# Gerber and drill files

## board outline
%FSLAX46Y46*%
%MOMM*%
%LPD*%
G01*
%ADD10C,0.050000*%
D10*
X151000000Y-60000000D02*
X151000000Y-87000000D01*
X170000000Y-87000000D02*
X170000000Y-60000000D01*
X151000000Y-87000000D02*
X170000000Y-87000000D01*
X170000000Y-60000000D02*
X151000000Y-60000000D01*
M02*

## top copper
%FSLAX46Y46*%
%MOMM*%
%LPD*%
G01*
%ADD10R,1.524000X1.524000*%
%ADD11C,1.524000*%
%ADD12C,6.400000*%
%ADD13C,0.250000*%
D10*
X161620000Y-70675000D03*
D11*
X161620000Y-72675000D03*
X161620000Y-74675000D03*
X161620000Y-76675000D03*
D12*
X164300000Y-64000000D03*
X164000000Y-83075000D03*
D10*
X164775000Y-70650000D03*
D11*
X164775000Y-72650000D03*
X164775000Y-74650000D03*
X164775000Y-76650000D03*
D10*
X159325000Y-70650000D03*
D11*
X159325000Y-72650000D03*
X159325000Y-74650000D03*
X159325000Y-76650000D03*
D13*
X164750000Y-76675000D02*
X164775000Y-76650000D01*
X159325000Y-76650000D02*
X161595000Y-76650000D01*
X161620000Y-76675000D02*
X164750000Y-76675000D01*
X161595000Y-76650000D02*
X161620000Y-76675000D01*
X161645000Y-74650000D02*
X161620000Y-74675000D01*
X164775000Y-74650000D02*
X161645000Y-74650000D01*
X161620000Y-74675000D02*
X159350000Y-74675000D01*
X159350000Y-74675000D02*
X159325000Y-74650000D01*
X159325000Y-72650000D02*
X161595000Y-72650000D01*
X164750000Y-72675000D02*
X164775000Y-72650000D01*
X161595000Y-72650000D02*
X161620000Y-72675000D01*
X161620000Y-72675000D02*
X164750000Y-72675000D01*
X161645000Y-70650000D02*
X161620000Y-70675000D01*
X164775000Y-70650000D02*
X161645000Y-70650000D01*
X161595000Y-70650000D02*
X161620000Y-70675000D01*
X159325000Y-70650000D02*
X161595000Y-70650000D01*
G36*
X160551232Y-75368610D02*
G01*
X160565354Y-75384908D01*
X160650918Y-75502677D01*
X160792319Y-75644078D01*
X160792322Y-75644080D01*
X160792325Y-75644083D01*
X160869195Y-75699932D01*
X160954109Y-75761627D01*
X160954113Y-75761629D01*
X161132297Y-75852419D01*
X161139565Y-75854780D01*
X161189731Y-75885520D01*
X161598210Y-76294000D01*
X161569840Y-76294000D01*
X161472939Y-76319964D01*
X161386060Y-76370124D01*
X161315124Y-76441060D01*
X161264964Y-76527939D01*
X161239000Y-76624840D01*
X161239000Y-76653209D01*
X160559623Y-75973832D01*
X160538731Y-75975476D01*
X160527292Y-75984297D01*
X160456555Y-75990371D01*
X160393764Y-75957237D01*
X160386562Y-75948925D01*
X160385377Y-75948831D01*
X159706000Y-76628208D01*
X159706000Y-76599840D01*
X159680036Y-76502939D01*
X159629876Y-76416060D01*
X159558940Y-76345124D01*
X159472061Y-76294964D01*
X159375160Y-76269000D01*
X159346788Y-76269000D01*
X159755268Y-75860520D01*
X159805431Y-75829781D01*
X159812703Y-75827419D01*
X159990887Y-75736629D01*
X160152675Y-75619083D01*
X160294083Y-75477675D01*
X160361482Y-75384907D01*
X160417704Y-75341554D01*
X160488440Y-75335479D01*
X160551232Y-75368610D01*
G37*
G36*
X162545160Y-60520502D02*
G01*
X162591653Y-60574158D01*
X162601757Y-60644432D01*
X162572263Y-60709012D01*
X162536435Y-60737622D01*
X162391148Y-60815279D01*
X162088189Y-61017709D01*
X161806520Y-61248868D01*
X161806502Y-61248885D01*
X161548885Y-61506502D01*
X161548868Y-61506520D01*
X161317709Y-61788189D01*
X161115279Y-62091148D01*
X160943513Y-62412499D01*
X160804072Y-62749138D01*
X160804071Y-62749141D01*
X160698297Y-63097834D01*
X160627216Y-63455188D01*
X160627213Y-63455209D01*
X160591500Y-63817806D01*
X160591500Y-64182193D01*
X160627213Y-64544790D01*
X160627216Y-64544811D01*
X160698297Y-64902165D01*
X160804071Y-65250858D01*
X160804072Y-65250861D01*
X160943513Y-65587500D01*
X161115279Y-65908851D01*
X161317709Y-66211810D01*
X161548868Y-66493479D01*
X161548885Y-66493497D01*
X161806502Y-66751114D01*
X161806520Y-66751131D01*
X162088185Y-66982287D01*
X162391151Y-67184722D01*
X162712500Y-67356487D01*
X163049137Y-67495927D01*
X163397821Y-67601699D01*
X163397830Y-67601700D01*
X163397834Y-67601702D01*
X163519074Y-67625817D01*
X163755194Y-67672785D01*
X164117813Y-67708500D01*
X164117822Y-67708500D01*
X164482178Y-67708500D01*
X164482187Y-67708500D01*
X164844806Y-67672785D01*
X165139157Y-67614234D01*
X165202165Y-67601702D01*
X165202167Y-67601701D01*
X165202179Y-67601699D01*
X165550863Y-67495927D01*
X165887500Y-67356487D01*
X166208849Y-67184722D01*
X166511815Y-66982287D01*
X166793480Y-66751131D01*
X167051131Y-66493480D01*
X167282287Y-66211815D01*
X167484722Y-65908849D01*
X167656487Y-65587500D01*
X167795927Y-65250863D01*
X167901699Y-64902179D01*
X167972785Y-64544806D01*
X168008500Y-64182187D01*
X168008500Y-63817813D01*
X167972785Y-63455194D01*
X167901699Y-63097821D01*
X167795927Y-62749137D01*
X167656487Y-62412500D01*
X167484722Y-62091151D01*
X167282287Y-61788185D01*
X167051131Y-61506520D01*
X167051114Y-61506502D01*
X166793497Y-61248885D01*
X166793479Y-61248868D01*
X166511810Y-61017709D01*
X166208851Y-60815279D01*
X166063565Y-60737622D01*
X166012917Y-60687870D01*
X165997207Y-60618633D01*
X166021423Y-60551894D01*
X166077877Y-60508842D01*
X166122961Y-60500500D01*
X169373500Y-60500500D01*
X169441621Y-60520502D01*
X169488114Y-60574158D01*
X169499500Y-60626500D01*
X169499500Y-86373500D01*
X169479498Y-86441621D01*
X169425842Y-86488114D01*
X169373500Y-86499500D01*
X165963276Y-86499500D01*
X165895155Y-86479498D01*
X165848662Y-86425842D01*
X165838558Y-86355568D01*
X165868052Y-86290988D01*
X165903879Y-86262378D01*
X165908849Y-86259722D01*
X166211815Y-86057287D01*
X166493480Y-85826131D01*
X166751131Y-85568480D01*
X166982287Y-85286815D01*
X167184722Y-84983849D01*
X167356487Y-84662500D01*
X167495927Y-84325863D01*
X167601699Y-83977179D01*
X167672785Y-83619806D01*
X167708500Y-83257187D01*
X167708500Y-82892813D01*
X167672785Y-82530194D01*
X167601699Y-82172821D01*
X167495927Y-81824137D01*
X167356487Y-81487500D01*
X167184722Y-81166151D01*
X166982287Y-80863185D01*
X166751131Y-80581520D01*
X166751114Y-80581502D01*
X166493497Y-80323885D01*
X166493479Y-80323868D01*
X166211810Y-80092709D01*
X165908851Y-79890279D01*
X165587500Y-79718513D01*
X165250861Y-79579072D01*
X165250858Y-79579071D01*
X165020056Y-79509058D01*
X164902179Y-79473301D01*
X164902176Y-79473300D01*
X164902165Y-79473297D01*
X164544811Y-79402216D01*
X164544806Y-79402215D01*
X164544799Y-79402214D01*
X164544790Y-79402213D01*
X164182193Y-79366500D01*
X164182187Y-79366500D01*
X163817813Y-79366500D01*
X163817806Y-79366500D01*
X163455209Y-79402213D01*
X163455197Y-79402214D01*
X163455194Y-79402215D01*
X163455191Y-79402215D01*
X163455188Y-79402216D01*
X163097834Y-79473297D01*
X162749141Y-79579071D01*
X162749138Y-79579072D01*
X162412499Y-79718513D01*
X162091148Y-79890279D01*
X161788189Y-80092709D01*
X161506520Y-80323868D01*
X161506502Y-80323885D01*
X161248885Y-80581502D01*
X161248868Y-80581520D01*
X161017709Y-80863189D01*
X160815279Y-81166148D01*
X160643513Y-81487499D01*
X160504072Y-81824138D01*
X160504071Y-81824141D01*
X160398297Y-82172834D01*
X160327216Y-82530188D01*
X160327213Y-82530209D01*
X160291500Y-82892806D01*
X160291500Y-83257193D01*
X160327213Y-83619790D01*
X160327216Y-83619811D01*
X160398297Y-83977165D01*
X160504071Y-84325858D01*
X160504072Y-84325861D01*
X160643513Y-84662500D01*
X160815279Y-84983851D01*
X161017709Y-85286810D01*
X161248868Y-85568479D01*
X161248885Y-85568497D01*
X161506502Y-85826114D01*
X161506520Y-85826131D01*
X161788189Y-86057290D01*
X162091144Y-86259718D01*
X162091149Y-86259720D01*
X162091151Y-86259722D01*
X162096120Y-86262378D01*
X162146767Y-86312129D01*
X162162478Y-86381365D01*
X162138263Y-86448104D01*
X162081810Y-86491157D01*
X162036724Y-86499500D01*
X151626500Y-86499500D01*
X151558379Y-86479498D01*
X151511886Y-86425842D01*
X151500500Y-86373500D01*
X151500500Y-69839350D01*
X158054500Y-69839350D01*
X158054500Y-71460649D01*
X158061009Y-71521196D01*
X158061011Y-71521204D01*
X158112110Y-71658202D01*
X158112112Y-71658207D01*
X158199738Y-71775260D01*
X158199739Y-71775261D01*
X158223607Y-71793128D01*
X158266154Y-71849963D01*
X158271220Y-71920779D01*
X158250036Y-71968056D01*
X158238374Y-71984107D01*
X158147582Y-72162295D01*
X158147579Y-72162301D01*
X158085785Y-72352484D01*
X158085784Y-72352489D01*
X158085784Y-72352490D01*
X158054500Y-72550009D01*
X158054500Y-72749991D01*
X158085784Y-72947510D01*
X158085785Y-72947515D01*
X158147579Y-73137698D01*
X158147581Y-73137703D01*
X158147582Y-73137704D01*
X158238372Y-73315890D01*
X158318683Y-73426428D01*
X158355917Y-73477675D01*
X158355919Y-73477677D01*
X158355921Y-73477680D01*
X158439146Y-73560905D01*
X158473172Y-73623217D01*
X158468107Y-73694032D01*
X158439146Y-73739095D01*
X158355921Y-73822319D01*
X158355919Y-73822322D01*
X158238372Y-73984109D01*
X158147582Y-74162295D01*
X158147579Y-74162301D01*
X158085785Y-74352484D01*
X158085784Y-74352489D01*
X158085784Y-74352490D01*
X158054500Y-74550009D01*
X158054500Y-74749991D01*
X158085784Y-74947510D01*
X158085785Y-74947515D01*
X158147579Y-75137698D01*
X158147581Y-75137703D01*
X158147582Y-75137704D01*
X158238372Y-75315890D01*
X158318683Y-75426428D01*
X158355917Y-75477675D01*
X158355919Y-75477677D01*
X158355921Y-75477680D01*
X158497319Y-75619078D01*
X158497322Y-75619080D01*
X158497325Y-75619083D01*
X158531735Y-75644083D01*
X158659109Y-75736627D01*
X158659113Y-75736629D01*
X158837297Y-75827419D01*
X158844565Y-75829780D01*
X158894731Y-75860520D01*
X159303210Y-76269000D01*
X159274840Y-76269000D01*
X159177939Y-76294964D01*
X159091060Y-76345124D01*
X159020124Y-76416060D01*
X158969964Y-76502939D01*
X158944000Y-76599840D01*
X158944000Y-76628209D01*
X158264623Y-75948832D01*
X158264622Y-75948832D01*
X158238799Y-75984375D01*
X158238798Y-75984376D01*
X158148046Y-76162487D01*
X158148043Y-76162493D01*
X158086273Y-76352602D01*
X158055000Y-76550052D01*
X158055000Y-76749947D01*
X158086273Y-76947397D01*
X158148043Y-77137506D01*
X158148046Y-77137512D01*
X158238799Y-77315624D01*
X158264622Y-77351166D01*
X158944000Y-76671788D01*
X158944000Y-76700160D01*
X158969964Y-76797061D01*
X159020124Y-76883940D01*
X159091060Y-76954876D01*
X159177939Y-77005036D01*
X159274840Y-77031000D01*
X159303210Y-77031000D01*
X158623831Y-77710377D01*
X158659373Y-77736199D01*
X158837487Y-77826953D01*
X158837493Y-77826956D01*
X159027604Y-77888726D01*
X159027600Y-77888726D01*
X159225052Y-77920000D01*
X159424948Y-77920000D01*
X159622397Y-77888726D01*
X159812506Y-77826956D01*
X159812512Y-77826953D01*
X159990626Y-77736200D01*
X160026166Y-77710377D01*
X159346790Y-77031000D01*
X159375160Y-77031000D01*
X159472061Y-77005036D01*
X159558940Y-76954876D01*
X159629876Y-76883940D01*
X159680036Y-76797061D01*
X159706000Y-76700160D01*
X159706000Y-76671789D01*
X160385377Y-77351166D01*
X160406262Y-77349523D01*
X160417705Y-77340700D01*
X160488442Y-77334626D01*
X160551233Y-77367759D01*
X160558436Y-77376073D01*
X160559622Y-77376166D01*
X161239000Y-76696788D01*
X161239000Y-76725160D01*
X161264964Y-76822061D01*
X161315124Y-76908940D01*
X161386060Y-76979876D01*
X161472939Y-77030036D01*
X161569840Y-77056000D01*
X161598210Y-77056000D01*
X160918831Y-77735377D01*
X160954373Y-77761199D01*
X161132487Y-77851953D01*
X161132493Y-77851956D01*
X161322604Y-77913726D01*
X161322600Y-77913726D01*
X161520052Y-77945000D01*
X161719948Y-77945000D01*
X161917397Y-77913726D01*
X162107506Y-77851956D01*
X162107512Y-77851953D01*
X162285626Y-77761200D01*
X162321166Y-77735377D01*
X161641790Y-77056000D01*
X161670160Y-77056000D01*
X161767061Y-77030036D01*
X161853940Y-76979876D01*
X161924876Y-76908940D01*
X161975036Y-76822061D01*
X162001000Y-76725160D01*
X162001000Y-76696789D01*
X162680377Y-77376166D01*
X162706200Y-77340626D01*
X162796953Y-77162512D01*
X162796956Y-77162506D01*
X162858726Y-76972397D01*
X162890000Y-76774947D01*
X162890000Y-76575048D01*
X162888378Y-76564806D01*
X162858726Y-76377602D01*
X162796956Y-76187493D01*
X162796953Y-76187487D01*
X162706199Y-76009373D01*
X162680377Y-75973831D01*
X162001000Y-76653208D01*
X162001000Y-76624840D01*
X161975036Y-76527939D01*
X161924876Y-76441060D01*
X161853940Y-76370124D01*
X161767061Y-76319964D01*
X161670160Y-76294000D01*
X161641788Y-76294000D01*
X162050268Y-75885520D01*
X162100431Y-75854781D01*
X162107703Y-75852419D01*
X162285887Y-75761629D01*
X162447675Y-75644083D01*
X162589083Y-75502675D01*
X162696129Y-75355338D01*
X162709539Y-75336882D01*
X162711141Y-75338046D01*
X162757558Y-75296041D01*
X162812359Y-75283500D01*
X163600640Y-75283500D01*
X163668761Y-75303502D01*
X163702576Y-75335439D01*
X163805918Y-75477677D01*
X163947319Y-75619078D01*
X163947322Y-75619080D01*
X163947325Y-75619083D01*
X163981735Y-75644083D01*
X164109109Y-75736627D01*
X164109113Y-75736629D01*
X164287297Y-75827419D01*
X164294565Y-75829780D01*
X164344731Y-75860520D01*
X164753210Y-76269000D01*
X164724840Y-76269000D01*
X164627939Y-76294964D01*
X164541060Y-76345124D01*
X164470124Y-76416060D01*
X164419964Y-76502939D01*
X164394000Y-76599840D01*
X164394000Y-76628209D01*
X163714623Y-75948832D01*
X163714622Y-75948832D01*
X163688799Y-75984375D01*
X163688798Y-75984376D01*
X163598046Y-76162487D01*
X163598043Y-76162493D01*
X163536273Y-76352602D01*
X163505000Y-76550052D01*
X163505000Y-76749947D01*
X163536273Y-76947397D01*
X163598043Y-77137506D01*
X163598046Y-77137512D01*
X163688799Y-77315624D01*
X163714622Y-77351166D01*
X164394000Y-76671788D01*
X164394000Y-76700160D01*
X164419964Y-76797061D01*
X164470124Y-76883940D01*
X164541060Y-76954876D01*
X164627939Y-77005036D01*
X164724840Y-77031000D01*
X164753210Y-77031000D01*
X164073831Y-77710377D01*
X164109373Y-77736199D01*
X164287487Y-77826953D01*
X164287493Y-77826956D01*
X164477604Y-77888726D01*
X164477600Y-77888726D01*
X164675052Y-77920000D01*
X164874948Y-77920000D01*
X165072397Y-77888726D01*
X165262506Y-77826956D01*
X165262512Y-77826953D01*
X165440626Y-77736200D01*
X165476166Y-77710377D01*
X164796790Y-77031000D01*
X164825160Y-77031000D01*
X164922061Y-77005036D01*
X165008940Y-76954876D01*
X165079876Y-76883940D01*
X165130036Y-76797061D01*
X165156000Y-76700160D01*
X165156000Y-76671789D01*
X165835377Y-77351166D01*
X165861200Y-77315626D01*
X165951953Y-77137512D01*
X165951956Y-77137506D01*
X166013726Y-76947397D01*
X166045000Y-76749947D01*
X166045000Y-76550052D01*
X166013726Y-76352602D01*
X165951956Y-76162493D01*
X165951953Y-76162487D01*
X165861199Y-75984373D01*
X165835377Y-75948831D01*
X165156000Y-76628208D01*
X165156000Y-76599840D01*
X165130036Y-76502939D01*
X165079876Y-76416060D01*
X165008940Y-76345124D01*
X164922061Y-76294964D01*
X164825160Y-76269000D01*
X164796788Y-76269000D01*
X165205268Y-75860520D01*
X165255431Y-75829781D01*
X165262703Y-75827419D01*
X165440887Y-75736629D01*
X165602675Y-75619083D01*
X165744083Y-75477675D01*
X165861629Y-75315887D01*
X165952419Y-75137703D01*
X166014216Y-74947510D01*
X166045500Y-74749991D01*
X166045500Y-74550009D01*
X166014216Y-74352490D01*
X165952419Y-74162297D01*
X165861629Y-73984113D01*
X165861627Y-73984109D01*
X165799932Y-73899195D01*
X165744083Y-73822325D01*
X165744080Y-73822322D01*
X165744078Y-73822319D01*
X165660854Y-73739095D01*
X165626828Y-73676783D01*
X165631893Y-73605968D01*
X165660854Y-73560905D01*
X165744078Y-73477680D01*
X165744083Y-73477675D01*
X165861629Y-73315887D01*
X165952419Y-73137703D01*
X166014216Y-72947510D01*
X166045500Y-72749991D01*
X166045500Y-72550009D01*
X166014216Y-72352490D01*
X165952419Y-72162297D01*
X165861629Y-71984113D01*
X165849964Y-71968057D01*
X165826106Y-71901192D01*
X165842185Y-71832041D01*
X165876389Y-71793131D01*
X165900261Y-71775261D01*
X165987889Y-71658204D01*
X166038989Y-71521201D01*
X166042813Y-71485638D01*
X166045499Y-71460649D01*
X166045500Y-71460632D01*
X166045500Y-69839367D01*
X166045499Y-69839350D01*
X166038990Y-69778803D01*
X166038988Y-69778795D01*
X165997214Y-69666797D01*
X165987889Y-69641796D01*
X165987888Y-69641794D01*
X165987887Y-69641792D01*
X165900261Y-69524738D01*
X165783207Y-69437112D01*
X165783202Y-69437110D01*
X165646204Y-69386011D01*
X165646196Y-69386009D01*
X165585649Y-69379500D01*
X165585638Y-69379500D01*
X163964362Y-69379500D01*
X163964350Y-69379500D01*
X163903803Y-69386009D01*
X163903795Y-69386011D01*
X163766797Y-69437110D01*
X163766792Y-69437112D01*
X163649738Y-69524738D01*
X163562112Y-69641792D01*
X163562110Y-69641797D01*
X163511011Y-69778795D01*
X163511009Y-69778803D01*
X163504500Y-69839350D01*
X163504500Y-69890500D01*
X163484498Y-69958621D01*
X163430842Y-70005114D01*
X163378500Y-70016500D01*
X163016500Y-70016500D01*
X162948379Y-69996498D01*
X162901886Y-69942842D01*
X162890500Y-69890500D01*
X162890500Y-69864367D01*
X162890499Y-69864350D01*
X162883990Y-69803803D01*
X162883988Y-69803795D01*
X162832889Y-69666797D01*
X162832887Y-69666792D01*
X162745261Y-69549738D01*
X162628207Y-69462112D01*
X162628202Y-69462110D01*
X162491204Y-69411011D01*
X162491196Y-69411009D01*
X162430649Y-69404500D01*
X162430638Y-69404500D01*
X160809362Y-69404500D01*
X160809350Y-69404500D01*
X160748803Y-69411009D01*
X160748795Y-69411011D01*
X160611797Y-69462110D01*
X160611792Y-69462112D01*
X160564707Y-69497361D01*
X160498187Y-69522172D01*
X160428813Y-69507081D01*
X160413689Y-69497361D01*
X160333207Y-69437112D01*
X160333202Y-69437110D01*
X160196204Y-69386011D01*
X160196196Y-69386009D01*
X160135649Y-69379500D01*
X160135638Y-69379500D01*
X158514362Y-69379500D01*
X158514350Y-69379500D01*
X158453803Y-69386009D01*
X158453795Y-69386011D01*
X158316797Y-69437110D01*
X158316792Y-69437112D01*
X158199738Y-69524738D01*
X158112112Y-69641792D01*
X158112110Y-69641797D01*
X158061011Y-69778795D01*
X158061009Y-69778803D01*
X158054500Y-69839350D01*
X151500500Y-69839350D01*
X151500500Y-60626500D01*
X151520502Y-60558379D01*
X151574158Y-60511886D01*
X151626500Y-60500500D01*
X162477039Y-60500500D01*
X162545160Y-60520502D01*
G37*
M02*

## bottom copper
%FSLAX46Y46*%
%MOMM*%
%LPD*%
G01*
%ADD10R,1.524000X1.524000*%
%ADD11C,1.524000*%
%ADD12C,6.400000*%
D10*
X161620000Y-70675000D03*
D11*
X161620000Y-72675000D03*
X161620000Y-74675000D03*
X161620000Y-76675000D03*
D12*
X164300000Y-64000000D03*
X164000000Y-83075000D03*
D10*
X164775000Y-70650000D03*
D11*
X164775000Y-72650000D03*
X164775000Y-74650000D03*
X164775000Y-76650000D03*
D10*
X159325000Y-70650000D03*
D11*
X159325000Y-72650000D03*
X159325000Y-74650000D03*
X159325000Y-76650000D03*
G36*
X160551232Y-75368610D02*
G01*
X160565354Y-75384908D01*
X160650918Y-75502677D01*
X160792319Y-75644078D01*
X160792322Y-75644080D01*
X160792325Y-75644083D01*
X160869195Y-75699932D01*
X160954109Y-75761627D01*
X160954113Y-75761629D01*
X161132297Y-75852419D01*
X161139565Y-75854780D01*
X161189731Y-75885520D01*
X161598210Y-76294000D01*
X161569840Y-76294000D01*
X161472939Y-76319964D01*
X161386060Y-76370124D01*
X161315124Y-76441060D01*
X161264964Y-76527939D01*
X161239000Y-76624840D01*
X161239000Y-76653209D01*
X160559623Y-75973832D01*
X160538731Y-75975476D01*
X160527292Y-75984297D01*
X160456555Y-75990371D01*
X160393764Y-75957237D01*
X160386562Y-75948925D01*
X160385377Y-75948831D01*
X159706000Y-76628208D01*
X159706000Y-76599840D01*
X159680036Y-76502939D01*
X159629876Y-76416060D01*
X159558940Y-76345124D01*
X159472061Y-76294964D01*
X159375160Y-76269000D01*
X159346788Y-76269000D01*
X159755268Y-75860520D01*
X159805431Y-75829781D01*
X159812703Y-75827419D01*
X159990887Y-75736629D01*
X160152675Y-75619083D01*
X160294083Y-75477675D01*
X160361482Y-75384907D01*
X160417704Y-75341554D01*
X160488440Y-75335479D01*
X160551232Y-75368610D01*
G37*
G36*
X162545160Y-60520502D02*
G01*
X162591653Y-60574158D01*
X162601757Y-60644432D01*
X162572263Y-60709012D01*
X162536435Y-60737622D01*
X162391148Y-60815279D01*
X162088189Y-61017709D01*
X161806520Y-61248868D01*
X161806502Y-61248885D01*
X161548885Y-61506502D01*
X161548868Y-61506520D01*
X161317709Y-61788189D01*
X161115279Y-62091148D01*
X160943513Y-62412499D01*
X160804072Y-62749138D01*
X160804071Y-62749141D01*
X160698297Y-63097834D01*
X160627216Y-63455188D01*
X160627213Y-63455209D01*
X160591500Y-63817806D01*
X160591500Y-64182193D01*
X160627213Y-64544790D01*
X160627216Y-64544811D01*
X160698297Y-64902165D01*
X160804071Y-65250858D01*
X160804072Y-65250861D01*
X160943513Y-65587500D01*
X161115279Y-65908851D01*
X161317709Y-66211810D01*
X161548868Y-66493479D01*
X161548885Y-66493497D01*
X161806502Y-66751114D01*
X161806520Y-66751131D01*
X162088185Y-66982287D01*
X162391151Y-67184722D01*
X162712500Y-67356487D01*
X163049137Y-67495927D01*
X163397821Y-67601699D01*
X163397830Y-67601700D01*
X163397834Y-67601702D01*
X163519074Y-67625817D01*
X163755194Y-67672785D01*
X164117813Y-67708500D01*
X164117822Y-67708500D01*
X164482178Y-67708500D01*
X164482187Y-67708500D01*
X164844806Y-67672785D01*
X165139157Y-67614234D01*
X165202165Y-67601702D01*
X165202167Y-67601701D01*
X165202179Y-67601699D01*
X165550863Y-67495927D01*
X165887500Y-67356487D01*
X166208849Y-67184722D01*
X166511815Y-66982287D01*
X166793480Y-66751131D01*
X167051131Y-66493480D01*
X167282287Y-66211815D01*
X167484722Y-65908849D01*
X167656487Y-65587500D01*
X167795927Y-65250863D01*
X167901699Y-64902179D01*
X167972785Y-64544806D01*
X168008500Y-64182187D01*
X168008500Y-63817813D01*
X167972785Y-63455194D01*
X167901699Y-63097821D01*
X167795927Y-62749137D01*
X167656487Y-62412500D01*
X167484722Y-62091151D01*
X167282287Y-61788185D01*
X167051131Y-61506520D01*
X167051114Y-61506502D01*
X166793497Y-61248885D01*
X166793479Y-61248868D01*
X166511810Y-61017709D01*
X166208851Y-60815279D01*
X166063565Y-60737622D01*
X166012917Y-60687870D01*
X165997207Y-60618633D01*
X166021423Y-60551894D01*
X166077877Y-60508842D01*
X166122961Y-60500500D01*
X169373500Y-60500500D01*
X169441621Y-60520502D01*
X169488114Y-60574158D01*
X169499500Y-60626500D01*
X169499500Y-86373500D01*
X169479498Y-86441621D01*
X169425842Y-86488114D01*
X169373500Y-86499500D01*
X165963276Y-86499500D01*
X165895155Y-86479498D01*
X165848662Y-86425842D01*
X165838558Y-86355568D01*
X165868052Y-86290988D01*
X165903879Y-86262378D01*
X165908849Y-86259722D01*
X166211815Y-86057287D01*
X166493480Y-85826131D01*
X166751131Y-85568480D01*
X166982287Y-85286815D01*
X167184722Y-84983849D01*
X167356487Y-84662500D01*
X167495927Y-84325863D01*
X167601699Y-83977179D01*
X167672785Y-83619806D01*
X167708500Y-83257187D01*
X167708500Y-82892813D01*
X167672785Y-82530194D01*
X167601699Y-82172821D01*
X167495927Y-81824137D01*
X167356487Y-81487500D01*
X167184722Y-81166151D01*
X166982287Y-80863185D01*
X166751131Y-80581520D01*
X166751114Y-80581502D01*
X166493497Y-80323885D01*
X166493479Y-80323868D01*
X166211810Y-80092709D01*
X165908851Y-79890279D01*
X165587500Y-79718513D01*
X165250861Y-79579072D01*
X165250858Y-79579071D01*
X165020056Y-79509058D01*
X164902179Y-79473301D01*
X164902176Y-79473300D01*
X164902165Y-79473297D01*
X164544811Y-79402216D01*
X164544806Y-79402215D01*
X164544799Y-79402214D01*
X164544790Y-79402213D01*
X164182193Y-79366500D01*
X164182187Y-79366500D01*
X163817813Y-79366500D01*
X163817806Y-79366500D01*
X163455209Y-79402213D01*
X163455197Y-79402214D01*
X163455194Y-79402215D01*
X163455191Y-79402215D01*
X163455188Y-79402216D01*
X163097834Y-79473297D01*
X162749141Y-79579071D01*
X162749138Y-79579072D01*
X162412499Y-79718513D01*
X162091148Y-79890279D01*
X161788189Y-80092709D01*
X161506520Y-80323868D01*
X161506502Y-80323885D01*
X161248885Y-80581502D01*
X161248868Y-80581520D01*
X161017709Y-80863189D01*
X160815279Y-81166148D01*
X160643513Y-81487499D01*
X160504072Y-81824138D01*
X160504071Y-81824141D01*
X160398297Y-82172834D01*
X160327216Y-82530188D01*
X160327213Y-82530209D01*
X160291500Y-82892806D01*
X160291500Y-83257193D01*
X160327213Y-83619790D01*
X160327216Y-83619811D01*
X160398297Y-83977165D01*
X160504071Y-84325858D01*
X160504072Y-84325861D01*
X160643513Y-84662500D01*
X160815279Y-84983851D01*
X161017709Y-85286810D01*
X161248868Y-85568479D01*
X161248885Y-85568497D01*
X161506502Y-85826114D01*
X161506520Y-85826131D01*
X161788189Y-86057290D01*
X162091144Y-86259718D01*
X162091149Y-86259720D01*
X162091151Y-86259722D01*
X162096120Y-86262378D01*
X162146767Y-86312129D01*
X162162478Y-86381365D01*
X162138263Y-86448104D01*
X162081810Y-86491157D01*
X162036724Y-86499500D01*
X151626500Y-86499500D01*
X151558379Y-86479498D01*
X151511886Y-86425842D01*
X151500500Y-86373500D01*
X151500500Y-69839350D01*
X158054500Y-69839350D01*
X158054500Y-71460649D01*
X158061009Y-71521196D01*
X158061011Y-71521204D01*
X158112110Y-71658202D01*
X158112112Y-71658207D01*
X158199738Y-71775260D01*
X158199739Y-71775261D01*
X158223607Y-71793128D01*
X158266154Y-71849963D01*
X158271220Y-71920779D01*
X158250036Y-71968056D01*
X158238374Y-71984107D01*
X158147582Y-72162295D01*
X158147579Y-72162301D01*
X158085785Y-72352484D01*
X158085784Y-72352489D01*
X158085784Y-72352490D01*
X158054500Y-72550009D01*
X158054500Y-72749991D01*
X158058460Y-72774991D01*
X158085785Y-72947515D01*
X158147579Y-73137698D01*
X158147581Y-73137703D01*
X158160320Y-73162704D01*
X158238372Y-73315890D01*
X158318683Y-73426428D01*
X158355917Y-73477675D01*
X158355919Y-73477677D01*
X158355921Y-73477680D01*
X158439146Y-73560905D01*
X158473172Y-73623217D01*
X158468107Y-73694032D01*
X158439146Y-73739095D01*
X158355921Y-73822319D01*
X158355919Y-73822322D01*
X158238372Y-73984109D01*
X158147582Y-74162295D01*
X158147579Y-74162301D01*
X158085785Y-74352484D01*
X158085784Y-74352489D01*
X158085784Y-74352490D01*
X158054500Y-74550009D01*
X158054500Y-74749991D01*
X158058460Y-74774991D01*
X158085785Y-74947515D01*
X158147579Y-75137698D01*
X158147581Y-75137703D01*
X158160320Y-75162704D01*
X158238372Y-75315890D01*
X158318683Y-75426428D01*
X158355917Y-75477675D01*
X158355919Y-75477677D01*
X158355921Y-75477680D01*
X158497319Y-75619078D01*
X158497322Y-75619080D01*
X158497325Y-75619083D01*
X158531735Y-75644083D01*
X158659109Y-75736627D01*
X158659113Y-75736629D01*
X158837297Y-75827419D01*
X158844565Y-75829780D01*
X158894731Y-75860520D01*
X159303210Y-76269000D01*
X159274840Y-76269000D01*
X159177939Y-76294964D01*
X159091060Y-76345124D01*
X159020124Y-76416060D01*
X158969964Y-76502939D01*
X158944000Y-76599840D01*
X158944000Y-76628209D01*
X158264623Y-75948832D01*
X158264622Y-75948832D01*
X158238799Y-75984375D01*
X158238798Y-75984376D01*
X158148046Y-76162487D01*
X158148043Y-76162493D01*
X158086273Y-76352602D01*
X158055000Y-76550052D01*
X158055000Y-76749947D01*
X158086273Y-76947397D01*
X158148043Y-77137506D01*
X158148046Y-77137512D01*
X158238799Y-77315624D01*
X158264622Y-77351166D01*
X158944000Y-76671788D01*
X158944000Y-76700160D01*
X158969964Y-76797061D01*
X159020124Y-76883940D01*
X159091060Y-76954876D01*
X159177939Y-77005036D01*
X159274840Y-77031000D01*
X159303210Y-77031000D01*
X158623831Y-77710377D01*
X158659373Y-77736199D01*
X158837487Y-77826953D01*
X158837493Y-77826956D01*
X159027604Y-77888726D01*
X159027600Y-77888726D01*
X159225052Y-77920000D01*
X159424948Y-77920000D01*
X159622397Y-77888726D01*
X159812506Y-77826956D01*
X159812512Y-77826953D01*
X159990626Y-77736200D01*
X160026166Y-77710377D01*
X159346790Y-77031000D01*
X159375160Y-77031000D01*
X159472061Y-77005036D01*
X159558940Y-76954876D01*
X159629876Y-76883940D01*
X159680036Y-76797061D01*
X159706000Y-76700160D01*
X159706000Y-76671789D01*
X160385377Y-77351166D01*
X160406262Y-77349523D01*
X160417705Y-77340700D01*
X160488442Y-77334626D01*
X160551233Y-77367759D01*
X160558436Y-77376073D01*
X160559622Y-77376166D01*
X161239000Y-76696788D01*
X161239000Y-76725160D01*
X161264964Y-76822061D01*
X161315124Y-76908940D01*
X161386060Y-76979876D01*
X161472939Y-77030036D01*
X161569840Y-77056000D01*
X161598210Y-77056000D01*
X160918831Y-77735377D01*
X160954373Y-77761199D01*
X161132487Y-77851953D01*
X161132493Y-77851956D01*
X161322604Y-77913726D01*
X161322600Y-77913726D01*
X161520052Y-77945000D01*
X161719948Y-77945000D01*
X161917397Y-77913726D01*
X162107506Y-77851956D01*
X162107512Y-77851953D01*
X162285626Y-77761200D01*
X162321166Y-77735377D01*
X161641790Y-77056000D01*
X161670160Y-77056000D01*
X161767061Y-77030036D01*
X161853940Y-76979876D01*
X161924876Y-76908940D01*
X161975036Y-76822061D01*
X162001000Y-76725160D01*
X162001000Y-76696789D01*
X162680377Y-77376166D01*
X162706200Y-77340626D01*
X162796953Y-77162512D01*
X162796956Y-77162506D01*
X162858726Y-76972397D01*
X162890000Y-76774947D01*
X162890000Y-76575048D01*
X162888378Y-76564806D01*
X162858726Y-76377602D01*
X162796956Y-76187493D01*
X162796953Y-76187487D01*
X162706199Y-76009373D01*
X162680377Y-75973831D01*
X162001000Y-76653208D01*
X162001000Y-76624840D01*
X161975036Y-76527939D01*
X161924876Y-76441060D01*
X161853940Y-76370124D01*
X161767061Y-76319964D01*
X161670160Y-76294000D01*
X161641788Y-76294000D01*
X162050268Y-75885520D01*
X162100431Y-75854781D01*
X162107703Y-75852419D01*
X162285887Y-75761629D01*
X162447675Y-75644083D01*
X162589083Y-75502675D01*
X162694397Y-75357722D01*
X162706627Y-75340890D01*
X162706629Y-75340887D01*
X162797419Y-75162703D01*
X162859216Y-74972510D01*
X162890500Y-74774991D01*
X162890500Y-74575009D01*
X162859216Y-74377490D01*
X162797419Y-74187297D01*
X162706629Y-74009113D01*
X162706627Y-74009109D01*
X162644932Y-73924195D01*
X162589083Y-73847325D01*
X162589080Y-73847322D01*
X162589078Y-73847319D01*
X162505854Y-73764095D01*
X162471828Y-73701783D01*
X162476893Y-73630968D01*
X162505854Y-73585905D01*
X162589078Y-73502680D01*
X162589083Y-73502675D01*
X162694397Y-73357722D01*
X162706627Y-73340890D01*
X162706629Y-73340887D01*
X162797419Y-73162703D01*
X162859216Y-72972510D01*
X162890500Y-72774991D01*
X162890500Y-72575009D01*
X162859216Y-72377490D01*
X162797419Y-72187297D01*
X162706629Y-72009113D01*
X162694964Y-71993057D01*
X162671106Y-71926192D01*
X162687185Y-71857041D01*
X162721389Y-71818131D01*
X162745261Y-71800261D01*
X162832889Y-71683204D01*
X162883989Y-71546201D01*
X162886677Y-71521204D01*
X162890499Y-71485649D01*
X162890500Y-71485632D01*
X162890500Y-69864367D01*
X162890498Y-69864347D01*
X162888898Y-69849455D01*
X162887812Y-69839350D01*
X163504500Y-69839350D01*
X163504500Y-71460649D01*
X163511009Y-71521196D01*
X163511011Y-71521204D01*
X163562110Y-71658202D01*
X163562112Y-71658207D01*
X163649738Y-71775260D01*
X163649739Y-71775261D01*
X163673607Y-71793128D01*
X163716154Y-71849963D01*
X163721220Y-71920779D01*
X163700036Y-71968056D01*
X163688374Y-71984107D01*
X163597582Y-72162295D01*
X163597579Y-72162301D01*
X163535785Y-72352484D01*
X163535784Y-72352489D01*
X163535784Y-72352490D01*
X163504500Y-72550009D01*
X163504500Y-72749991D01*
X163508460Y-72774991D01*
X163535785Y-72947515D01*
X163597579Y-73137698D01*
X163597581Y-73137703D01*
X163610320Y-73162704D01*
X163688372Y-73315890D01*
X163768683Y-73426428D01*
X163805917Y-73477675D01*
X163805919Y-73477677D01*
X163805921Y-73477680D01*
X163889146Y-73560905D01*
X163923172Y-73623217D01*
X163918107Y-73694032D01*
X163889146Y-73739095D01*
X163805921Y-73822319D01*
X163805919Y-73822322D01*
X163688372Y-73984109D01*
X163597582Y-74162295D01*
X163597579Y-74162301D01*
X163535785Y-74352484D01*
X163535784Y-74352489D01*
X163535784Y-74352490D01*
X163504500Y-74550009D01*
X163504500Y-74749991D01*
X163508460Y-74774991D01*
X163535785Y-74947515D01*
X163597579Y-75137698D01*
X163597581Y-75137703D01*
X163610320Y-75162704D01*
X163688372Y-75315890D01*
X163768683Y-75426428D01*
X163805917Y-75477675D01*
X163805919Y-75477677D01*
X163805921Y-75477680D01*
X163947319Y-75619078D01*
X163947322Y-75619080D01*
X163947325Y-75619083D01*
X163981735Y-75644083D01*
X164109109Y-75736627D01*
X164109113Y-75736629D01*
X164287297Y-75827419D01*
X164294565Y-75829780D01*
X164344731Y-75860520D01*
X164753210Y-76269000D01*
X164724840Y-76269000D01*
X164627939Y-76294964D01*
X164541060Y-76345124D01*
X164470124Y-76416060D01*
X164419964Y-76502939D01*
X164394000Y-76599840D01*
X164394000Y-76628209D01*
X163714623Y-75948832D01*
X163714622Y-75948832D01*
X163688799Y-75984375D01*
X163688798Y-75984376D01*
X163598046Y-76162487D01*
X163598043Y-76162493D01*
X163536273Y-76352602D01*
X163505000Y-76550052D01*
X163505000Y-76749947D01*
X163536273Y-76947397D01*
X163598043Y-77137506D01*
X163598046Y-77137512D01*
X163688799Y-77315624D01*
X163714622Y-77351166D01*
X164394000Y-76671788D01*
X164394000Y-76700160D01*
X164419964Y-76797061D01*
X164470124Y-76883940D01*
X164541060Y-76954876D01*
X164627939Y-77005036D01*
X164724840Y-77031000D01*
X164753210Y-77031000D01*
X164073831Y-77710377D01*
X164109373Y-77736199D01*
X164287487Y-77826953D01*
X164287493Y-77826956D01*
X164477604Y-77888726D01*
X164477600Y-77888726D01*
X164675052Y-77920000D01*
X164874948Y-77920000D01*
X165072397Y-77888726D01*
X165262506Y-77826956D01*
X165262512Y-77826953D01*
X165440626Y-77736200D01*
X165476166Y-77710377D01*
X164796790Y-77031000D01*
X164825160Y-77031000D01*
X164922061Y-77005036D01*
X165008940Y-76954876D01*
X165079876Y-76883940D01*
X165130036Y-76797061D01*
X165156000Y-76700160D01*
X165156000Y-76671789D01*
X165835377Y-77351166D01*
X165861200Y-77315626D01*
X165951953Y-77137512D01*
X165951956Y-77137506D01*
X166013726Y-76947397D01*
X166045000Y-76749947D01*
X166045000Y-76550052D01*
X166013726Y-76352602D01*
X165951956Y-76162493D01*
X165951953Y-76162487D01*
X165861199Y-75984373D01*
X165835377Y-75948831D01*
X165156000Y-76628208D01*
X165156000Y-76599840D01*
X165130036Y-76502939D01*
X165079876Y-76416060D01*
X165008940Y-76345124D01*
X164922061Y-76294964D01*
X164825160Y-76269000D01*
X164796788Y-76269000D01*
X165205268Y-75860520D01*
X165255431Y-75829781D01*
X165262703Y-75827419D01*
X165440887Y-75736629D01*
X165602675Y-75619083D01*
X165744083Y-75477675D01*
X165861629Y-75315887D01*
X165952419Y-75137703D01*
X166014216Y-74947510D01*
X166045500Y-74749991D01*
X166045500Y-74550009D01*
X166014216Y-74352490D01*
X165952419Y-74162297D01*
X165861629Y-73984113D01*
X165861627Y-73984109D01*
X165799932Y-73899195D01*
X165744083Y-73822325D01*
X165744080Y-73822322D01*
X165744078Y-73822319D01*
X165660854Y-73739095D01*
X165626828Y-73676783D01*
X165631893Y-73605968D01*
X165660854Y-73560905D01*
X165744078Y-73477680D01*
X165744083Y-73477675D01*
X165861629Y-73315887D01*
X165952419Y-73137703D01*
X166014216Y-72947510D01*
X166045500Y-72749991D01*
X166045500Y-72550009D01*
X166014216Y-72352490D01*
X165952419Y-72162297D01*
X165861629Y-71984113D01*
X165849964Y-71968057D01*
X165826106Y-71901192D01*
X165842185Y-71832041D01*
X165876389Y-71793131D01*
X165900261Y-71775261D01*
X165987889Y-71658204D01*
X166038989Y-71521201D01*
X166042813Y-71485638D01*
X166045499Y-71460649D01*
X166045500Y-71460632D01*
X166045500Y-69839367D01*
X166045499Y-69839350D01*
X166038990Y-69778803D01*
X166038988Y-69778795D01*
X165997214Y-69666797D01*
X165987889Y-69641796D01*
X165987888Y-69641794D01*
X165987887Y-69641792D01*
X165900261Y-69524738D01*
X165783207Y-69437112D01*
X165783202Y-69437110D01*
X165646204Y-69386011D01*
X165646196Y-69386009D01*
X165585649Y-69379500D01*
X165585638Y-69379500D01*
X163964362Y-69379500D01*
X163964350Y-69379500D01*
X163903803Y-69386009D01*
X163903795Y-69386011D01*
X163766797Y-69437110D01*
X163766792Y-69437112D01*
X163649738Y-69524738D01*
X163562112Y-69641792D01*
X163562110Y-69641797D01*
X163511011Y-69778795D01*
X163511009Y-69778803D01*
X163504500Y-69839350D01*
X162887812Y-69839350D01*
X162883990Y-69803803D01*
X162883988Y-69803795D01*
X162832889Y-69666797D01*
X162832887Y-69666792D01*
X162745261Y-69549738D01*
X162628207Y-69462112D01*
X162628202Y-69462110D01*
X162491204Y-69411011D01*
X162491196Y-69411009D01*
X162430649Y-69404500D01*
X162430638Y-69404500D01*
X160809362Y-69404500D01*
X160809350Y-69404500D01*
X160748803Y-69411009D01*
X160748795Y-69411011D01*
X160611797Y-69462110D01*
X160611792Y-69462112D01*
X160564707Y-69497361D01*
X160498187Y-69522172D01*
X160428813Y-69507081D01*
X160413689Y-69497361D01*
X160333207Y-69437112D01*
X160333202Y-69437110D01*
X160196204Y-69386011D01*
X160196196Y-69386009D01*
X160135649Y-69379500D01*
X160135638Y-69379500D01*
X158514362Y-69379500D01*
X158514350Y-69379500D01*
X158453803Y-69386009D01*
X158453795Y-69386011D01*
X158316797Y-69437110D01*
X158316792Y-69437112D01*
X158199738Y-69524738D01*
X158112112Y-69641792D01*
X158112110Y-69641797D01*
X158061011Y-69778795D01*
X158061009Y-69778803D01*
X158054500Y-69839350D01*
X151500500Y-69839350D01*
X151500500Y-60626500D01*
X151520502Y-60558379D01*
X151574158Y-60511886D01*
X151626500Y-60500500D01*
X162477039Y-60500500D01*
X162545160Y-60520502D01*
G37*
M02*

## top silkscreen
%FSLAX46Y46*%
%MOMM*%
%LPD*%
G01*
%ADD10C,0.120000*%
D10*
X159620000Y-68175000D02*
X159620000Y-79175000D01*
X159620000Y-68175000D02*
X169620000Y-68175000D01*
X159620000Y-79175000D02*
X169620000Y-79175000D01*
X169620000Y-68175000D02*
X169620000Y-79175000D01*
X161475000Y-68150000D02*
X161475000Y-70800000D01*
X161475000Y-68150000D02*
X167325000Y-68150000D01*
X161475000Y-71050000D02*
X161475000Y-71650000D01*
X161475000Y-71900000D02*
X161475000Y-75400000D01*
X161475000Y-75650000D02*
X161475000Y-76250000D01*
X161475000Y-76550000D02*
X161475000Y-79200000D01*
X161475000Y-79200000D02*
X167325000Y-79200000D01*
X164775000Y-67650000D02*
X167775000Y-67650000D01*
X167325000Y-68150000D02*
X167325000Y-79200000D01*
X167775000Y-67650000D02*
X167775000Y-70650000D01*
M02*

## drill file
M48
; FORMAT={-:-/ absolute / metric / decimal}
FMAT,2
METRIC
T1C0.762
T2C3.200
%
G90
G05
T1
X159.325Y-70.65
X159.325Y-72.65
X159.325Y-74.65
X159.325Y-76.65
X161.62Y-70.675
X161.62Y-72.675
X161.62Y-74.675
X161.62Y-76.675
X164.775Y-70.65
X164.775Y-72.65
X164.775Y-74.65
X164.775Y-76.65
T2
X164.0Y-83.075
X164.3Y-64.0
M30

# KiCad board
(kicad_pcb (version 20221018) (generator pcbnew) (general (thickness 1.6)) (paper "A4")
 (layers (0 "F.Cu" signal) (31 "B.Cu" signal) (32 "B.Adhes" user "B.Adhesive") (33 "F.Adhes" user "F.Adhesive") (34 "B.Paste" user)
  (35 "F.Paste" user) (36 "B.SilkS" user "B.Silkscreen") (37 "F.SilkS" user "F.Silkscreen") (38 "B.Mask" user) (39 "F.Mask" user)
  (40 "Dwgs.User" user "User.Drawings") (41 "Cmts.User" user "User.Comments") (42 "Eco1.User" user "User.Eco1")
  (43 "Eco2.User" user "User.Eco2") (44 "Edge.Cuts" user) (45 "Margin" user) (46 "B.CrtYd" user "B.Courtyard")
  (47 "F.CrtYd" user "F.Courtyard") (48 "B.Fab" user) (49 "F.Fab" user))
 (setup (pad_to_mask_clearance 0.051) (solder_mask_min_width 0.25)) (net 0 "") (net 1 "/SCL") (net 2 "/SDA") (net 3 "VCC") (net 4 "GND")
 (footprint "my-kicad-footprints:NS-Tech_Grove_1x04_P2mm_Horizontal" (layer "F.Cu") (at 161.62 73.675)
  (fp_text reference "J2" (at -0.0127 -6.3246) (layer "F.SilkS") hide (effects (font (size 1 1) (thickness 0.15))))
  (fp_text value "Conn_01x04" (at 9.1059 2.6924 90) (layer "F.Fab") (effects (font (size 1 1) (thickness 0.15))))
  (fp_line (start -2 -5.5) (end -2 5.5) (stroke (width 0.12) (type solid)) (layer "F.SilkS"))
  (fp_line (start -2 -5.5) (end 8 -5.5) (stroke (width 0.12) (type solid)) (layer "F.SilkS"))
  (fp_line (start -2 5.5) (end 8 5.5) (stroke (width 0.12) (type solid)) (layer "F.SilkS"))
  (fp_line (start 8 -5.5) (end 8 5.5) (stroke (width 0.12) (type solid)) (layer "F.SilkS"))
  (pad "1" thru_hole rect (at 0 -3) (size 1.524 1.524) (drill 0.762) (layers "*.Cu" "*.Mask") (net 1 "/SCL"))
  (pad "2" thru_hole circle (at 0 -1) (size 1.524 1.524) (drill 0.762) (layers "*.Cu" "*.Mask") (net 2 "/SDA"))
  (pad "3" thru_hole circle (at 0 1) (size 1.524 1.524) (drill 0.762) (layers "*.Cu" "*.Mask") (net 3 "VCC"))
  (pad "4" thru_hole circle (at 0 3) (size 1.524 1.524) (drill 0.762) (layers "*.Cu" "*.Mask") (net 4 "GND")))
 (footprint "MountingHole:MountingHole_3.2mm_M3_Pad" (layer "F.Cu") (at 164.3 64)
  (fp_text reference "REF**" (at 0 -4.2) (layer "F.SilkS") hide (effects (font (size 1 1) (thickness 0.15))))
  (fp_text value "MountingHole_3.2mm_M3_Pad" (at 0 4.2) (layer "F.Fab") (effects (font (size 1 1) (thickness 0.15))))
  (pad "1" thru_hole circle (at 0 0) (size 6.4 6.4) (drill 3.2) (layers "*.Cu" "*.Mask")))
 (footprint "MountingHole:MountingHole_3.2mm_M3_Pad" (layer "F.Cu") (at 164 83.075)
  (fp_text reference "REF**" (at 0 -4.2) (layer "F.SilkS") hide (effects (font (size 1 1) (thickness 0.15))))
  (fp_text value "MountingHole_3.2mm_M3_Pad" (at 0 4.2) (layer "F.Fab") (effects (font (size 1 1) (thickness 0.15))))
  (pad "1" thru_hole circle (at 0 0) (size 6.4 6.4) (drill 3.2) (layers "*.Cu" "*.Mask")))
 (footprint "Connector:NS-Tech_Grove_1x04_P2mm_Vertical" (layer "F.Cu") (at 164.775 70.65)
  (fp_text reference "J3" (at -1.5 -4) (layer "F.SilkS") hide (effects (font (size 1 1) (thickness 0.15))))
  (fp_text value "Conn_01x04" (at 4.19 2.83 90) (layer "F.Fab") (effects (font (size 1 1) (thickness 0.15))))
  (fp_line (start -3.3 -2.5) (end -3.3 0.15) (stroke (width 0.12) (type solid)) (layer "F.SilkS"))
  (fp_line (start -3.3 -2.5) (end 2.55 -2.5) (stroke (width 0.12) (type solid)) (layer "F.SilkS"))
  (fp_line (start -3.3 0.4) (end -3.3 1) (stroke (width 0.12) (type solid)) (layer "F.SilkS"))
  (fp_line (start -3.3 1.25) (end -3.3 4.75) (stroke (width 0.12) (type solid)) (layer "F.SilkS"))
  (fp_line (start -3.3 5) (end -3.3 5.6) (stroke (width 0.12) (type solid)) (layer "F.SilkS"))
  (fp_line (start -3.3 5.9) (end -3.3 8.55) (stroke (width 0.12) (type solid)) (layer "F.SilkS"))
  (fp_line (start -3.3 8.55) (end 2.55 8.55) (stroke (width 0.12) (type solid)) (layer "F.SilkS"))
  (fp_line (start 0 -3) (end 3 -3) (stroke (width 0.12) (type solid)) (layer "F.SilkS"))
  (fp_line (start 2.55 -2.5) (end 2.55 8.55) (stroke (width 0.12) (type solid)) (layer "F.SilkS"))
  (fp_line (start 3 -3) (end 3 0) (stroke (width 0.12) (type solid)) (layer "F.SilkS"))
  (pad "1" thru_hole rect (at 0 0) (size 1.524 1.524) (drill 0.762) (layers "*.Cu" "*.Mask") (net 1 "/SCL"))
  (pad "2" thru_hole circle (at 0 2) (size 1.524 1.524) (drill 0.762) (layers "*.Cu" "*.Mask") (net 2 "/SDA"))
  (pad "3" thru_hole circle (at 0 4) (size 1.524 1.524) (drill 0.762) (layers "*.Cu" "*.Mask") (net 3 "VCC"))
  (pad "4" thru_hole circle (at 0 6) (size 1.524 1.524) (drill 0.762) (layers "*.Cu" "*.Mask") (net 4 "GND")))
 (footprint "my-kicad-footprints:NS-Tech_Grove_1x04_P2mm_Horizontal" (layer "B.Cu") (at 159.325 73.65 180)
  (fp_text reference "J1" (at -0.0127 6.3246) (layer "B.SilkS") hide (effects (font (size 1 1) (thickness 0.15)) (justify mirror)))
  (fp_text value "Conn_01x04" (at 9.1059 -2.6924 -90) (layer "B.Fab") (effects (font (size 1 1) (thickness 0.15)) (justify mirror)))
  (pad "1" thru_hole rect (at 0 3 180) (size 1.524 1.524) (drill 0.762) (layers "*.Cu" "*.Mask") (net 1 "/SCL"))
  (pad "2" thru_hole circle (at 0 1 180) (size 1.524 1.524) (drill 0.762) (layers "*.Cu" "*.Mask") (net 2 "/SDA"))
  (pad "3" thru_hole circle (at 0 -1 180) (size 1.524 1.524) (drill 0.762) (layers "*.Cu" "*.Mask") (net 3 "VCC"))
  (pad "4" thru_hole circle (at 0 -3 180) (size 1.524 1.524) (drill 0.762) (layers "*.Cu" "*.Mask") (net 4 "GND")))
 (gr_line (start 151 60) (end 151 87) (stroke (width 0.05) (type solid)) (layer "Edge.Cuts"))
 (gr_line (start 170 87) (end 170 60) (stroke (width 0.05) (type solid)) (layer "Edge.Cuts"))
 (gr_line (start 151 87) (end 170 87) (stroke (width 0.05) (type solid)) (layer "Edge.Cuts"))
 (gr_line (start 170 60) (end 151 60) (stroke (width 0.05) (type solid)) (layer "Edge.Cuts"))
 (segment (start 164.75 76.675) (end 164.775 76.65) (width 0.25) (layer "F.Cu") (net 4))
 (segment (start 159.325 76.65) (end 161.595 76.65) (width 0.25) (layer "F.Cu") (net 4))
 (segment (start 161.62 76.675) (end 164.75 76.675) (width 0.25) (layer "F.Cu") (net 4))
 (segment (start 161.595 76.65) (end 161.62 76.675) (width 0.25) (layer "F.Cu") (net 4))
 (segment (start 161.645 74.65) (end 161.62 74.675) (width 0.25) (layer "F.Cu") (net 3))
 (segment (start 164.775 74.65) (end 161.645 74.65) (width 0.25) (layer "F.Cu") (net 3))
 (segment (start 161.62 74.675) (end 159.35 74.675) (width 0.25) (layer "F.Cu") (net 3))
 (segment (start 159.35 74.675) (end 159.325 74.65) (width 0.25) (layer "F.Cu") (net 3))
 (segment (start 159.325 72.65) (end 161.595 72.65) (width 0.25) (layer "F.Cu") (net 2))
 (segment (start 164.75 72.675) (end 164.775 72.65) (width 0.25) (layer "F.Cu") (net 2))
 (segment (start 161.595 72.65) (end 161.62 72.675) (width 0.25) (layer "F.Cu") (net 2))
 (segment (start 161.62 72.675) (end 164.75 72.675) (width 0.25) (layer "F.Cu") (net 2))
 (segment (start 161.645 70.65) (end 161.62 70.675) (width 0.25) (layer "F.Cu") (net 1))
 (segment (start 164.775 70.65) (end 161.645 70.65) (width 0.25) (layer "F.Cu") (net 1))
 (segment (start 161.595 70.65) (end 161.62 70.675) (width 0.25) (layer "F.Cu") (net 1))
 (segment (start 159.325 70.65) (end 161.595 70.65) (width 0.25) (layer "F.Cu") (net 1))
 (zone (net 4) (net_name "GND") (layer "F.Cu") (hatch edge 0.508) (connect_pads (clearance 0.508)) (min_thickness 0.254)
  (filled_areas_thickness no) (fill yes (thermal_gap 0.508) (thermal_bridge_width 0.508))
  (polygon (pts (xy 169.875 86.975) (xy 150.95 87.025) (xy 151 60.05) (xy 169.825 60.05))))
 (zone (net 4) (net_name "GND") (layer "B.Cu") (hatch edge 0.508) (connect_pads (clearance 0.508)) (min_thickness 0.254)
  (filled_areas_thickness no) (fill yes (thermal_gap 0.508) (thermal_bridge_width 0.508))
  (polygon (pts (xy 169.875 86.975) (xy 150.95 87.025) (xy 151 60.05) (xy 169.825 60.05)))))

